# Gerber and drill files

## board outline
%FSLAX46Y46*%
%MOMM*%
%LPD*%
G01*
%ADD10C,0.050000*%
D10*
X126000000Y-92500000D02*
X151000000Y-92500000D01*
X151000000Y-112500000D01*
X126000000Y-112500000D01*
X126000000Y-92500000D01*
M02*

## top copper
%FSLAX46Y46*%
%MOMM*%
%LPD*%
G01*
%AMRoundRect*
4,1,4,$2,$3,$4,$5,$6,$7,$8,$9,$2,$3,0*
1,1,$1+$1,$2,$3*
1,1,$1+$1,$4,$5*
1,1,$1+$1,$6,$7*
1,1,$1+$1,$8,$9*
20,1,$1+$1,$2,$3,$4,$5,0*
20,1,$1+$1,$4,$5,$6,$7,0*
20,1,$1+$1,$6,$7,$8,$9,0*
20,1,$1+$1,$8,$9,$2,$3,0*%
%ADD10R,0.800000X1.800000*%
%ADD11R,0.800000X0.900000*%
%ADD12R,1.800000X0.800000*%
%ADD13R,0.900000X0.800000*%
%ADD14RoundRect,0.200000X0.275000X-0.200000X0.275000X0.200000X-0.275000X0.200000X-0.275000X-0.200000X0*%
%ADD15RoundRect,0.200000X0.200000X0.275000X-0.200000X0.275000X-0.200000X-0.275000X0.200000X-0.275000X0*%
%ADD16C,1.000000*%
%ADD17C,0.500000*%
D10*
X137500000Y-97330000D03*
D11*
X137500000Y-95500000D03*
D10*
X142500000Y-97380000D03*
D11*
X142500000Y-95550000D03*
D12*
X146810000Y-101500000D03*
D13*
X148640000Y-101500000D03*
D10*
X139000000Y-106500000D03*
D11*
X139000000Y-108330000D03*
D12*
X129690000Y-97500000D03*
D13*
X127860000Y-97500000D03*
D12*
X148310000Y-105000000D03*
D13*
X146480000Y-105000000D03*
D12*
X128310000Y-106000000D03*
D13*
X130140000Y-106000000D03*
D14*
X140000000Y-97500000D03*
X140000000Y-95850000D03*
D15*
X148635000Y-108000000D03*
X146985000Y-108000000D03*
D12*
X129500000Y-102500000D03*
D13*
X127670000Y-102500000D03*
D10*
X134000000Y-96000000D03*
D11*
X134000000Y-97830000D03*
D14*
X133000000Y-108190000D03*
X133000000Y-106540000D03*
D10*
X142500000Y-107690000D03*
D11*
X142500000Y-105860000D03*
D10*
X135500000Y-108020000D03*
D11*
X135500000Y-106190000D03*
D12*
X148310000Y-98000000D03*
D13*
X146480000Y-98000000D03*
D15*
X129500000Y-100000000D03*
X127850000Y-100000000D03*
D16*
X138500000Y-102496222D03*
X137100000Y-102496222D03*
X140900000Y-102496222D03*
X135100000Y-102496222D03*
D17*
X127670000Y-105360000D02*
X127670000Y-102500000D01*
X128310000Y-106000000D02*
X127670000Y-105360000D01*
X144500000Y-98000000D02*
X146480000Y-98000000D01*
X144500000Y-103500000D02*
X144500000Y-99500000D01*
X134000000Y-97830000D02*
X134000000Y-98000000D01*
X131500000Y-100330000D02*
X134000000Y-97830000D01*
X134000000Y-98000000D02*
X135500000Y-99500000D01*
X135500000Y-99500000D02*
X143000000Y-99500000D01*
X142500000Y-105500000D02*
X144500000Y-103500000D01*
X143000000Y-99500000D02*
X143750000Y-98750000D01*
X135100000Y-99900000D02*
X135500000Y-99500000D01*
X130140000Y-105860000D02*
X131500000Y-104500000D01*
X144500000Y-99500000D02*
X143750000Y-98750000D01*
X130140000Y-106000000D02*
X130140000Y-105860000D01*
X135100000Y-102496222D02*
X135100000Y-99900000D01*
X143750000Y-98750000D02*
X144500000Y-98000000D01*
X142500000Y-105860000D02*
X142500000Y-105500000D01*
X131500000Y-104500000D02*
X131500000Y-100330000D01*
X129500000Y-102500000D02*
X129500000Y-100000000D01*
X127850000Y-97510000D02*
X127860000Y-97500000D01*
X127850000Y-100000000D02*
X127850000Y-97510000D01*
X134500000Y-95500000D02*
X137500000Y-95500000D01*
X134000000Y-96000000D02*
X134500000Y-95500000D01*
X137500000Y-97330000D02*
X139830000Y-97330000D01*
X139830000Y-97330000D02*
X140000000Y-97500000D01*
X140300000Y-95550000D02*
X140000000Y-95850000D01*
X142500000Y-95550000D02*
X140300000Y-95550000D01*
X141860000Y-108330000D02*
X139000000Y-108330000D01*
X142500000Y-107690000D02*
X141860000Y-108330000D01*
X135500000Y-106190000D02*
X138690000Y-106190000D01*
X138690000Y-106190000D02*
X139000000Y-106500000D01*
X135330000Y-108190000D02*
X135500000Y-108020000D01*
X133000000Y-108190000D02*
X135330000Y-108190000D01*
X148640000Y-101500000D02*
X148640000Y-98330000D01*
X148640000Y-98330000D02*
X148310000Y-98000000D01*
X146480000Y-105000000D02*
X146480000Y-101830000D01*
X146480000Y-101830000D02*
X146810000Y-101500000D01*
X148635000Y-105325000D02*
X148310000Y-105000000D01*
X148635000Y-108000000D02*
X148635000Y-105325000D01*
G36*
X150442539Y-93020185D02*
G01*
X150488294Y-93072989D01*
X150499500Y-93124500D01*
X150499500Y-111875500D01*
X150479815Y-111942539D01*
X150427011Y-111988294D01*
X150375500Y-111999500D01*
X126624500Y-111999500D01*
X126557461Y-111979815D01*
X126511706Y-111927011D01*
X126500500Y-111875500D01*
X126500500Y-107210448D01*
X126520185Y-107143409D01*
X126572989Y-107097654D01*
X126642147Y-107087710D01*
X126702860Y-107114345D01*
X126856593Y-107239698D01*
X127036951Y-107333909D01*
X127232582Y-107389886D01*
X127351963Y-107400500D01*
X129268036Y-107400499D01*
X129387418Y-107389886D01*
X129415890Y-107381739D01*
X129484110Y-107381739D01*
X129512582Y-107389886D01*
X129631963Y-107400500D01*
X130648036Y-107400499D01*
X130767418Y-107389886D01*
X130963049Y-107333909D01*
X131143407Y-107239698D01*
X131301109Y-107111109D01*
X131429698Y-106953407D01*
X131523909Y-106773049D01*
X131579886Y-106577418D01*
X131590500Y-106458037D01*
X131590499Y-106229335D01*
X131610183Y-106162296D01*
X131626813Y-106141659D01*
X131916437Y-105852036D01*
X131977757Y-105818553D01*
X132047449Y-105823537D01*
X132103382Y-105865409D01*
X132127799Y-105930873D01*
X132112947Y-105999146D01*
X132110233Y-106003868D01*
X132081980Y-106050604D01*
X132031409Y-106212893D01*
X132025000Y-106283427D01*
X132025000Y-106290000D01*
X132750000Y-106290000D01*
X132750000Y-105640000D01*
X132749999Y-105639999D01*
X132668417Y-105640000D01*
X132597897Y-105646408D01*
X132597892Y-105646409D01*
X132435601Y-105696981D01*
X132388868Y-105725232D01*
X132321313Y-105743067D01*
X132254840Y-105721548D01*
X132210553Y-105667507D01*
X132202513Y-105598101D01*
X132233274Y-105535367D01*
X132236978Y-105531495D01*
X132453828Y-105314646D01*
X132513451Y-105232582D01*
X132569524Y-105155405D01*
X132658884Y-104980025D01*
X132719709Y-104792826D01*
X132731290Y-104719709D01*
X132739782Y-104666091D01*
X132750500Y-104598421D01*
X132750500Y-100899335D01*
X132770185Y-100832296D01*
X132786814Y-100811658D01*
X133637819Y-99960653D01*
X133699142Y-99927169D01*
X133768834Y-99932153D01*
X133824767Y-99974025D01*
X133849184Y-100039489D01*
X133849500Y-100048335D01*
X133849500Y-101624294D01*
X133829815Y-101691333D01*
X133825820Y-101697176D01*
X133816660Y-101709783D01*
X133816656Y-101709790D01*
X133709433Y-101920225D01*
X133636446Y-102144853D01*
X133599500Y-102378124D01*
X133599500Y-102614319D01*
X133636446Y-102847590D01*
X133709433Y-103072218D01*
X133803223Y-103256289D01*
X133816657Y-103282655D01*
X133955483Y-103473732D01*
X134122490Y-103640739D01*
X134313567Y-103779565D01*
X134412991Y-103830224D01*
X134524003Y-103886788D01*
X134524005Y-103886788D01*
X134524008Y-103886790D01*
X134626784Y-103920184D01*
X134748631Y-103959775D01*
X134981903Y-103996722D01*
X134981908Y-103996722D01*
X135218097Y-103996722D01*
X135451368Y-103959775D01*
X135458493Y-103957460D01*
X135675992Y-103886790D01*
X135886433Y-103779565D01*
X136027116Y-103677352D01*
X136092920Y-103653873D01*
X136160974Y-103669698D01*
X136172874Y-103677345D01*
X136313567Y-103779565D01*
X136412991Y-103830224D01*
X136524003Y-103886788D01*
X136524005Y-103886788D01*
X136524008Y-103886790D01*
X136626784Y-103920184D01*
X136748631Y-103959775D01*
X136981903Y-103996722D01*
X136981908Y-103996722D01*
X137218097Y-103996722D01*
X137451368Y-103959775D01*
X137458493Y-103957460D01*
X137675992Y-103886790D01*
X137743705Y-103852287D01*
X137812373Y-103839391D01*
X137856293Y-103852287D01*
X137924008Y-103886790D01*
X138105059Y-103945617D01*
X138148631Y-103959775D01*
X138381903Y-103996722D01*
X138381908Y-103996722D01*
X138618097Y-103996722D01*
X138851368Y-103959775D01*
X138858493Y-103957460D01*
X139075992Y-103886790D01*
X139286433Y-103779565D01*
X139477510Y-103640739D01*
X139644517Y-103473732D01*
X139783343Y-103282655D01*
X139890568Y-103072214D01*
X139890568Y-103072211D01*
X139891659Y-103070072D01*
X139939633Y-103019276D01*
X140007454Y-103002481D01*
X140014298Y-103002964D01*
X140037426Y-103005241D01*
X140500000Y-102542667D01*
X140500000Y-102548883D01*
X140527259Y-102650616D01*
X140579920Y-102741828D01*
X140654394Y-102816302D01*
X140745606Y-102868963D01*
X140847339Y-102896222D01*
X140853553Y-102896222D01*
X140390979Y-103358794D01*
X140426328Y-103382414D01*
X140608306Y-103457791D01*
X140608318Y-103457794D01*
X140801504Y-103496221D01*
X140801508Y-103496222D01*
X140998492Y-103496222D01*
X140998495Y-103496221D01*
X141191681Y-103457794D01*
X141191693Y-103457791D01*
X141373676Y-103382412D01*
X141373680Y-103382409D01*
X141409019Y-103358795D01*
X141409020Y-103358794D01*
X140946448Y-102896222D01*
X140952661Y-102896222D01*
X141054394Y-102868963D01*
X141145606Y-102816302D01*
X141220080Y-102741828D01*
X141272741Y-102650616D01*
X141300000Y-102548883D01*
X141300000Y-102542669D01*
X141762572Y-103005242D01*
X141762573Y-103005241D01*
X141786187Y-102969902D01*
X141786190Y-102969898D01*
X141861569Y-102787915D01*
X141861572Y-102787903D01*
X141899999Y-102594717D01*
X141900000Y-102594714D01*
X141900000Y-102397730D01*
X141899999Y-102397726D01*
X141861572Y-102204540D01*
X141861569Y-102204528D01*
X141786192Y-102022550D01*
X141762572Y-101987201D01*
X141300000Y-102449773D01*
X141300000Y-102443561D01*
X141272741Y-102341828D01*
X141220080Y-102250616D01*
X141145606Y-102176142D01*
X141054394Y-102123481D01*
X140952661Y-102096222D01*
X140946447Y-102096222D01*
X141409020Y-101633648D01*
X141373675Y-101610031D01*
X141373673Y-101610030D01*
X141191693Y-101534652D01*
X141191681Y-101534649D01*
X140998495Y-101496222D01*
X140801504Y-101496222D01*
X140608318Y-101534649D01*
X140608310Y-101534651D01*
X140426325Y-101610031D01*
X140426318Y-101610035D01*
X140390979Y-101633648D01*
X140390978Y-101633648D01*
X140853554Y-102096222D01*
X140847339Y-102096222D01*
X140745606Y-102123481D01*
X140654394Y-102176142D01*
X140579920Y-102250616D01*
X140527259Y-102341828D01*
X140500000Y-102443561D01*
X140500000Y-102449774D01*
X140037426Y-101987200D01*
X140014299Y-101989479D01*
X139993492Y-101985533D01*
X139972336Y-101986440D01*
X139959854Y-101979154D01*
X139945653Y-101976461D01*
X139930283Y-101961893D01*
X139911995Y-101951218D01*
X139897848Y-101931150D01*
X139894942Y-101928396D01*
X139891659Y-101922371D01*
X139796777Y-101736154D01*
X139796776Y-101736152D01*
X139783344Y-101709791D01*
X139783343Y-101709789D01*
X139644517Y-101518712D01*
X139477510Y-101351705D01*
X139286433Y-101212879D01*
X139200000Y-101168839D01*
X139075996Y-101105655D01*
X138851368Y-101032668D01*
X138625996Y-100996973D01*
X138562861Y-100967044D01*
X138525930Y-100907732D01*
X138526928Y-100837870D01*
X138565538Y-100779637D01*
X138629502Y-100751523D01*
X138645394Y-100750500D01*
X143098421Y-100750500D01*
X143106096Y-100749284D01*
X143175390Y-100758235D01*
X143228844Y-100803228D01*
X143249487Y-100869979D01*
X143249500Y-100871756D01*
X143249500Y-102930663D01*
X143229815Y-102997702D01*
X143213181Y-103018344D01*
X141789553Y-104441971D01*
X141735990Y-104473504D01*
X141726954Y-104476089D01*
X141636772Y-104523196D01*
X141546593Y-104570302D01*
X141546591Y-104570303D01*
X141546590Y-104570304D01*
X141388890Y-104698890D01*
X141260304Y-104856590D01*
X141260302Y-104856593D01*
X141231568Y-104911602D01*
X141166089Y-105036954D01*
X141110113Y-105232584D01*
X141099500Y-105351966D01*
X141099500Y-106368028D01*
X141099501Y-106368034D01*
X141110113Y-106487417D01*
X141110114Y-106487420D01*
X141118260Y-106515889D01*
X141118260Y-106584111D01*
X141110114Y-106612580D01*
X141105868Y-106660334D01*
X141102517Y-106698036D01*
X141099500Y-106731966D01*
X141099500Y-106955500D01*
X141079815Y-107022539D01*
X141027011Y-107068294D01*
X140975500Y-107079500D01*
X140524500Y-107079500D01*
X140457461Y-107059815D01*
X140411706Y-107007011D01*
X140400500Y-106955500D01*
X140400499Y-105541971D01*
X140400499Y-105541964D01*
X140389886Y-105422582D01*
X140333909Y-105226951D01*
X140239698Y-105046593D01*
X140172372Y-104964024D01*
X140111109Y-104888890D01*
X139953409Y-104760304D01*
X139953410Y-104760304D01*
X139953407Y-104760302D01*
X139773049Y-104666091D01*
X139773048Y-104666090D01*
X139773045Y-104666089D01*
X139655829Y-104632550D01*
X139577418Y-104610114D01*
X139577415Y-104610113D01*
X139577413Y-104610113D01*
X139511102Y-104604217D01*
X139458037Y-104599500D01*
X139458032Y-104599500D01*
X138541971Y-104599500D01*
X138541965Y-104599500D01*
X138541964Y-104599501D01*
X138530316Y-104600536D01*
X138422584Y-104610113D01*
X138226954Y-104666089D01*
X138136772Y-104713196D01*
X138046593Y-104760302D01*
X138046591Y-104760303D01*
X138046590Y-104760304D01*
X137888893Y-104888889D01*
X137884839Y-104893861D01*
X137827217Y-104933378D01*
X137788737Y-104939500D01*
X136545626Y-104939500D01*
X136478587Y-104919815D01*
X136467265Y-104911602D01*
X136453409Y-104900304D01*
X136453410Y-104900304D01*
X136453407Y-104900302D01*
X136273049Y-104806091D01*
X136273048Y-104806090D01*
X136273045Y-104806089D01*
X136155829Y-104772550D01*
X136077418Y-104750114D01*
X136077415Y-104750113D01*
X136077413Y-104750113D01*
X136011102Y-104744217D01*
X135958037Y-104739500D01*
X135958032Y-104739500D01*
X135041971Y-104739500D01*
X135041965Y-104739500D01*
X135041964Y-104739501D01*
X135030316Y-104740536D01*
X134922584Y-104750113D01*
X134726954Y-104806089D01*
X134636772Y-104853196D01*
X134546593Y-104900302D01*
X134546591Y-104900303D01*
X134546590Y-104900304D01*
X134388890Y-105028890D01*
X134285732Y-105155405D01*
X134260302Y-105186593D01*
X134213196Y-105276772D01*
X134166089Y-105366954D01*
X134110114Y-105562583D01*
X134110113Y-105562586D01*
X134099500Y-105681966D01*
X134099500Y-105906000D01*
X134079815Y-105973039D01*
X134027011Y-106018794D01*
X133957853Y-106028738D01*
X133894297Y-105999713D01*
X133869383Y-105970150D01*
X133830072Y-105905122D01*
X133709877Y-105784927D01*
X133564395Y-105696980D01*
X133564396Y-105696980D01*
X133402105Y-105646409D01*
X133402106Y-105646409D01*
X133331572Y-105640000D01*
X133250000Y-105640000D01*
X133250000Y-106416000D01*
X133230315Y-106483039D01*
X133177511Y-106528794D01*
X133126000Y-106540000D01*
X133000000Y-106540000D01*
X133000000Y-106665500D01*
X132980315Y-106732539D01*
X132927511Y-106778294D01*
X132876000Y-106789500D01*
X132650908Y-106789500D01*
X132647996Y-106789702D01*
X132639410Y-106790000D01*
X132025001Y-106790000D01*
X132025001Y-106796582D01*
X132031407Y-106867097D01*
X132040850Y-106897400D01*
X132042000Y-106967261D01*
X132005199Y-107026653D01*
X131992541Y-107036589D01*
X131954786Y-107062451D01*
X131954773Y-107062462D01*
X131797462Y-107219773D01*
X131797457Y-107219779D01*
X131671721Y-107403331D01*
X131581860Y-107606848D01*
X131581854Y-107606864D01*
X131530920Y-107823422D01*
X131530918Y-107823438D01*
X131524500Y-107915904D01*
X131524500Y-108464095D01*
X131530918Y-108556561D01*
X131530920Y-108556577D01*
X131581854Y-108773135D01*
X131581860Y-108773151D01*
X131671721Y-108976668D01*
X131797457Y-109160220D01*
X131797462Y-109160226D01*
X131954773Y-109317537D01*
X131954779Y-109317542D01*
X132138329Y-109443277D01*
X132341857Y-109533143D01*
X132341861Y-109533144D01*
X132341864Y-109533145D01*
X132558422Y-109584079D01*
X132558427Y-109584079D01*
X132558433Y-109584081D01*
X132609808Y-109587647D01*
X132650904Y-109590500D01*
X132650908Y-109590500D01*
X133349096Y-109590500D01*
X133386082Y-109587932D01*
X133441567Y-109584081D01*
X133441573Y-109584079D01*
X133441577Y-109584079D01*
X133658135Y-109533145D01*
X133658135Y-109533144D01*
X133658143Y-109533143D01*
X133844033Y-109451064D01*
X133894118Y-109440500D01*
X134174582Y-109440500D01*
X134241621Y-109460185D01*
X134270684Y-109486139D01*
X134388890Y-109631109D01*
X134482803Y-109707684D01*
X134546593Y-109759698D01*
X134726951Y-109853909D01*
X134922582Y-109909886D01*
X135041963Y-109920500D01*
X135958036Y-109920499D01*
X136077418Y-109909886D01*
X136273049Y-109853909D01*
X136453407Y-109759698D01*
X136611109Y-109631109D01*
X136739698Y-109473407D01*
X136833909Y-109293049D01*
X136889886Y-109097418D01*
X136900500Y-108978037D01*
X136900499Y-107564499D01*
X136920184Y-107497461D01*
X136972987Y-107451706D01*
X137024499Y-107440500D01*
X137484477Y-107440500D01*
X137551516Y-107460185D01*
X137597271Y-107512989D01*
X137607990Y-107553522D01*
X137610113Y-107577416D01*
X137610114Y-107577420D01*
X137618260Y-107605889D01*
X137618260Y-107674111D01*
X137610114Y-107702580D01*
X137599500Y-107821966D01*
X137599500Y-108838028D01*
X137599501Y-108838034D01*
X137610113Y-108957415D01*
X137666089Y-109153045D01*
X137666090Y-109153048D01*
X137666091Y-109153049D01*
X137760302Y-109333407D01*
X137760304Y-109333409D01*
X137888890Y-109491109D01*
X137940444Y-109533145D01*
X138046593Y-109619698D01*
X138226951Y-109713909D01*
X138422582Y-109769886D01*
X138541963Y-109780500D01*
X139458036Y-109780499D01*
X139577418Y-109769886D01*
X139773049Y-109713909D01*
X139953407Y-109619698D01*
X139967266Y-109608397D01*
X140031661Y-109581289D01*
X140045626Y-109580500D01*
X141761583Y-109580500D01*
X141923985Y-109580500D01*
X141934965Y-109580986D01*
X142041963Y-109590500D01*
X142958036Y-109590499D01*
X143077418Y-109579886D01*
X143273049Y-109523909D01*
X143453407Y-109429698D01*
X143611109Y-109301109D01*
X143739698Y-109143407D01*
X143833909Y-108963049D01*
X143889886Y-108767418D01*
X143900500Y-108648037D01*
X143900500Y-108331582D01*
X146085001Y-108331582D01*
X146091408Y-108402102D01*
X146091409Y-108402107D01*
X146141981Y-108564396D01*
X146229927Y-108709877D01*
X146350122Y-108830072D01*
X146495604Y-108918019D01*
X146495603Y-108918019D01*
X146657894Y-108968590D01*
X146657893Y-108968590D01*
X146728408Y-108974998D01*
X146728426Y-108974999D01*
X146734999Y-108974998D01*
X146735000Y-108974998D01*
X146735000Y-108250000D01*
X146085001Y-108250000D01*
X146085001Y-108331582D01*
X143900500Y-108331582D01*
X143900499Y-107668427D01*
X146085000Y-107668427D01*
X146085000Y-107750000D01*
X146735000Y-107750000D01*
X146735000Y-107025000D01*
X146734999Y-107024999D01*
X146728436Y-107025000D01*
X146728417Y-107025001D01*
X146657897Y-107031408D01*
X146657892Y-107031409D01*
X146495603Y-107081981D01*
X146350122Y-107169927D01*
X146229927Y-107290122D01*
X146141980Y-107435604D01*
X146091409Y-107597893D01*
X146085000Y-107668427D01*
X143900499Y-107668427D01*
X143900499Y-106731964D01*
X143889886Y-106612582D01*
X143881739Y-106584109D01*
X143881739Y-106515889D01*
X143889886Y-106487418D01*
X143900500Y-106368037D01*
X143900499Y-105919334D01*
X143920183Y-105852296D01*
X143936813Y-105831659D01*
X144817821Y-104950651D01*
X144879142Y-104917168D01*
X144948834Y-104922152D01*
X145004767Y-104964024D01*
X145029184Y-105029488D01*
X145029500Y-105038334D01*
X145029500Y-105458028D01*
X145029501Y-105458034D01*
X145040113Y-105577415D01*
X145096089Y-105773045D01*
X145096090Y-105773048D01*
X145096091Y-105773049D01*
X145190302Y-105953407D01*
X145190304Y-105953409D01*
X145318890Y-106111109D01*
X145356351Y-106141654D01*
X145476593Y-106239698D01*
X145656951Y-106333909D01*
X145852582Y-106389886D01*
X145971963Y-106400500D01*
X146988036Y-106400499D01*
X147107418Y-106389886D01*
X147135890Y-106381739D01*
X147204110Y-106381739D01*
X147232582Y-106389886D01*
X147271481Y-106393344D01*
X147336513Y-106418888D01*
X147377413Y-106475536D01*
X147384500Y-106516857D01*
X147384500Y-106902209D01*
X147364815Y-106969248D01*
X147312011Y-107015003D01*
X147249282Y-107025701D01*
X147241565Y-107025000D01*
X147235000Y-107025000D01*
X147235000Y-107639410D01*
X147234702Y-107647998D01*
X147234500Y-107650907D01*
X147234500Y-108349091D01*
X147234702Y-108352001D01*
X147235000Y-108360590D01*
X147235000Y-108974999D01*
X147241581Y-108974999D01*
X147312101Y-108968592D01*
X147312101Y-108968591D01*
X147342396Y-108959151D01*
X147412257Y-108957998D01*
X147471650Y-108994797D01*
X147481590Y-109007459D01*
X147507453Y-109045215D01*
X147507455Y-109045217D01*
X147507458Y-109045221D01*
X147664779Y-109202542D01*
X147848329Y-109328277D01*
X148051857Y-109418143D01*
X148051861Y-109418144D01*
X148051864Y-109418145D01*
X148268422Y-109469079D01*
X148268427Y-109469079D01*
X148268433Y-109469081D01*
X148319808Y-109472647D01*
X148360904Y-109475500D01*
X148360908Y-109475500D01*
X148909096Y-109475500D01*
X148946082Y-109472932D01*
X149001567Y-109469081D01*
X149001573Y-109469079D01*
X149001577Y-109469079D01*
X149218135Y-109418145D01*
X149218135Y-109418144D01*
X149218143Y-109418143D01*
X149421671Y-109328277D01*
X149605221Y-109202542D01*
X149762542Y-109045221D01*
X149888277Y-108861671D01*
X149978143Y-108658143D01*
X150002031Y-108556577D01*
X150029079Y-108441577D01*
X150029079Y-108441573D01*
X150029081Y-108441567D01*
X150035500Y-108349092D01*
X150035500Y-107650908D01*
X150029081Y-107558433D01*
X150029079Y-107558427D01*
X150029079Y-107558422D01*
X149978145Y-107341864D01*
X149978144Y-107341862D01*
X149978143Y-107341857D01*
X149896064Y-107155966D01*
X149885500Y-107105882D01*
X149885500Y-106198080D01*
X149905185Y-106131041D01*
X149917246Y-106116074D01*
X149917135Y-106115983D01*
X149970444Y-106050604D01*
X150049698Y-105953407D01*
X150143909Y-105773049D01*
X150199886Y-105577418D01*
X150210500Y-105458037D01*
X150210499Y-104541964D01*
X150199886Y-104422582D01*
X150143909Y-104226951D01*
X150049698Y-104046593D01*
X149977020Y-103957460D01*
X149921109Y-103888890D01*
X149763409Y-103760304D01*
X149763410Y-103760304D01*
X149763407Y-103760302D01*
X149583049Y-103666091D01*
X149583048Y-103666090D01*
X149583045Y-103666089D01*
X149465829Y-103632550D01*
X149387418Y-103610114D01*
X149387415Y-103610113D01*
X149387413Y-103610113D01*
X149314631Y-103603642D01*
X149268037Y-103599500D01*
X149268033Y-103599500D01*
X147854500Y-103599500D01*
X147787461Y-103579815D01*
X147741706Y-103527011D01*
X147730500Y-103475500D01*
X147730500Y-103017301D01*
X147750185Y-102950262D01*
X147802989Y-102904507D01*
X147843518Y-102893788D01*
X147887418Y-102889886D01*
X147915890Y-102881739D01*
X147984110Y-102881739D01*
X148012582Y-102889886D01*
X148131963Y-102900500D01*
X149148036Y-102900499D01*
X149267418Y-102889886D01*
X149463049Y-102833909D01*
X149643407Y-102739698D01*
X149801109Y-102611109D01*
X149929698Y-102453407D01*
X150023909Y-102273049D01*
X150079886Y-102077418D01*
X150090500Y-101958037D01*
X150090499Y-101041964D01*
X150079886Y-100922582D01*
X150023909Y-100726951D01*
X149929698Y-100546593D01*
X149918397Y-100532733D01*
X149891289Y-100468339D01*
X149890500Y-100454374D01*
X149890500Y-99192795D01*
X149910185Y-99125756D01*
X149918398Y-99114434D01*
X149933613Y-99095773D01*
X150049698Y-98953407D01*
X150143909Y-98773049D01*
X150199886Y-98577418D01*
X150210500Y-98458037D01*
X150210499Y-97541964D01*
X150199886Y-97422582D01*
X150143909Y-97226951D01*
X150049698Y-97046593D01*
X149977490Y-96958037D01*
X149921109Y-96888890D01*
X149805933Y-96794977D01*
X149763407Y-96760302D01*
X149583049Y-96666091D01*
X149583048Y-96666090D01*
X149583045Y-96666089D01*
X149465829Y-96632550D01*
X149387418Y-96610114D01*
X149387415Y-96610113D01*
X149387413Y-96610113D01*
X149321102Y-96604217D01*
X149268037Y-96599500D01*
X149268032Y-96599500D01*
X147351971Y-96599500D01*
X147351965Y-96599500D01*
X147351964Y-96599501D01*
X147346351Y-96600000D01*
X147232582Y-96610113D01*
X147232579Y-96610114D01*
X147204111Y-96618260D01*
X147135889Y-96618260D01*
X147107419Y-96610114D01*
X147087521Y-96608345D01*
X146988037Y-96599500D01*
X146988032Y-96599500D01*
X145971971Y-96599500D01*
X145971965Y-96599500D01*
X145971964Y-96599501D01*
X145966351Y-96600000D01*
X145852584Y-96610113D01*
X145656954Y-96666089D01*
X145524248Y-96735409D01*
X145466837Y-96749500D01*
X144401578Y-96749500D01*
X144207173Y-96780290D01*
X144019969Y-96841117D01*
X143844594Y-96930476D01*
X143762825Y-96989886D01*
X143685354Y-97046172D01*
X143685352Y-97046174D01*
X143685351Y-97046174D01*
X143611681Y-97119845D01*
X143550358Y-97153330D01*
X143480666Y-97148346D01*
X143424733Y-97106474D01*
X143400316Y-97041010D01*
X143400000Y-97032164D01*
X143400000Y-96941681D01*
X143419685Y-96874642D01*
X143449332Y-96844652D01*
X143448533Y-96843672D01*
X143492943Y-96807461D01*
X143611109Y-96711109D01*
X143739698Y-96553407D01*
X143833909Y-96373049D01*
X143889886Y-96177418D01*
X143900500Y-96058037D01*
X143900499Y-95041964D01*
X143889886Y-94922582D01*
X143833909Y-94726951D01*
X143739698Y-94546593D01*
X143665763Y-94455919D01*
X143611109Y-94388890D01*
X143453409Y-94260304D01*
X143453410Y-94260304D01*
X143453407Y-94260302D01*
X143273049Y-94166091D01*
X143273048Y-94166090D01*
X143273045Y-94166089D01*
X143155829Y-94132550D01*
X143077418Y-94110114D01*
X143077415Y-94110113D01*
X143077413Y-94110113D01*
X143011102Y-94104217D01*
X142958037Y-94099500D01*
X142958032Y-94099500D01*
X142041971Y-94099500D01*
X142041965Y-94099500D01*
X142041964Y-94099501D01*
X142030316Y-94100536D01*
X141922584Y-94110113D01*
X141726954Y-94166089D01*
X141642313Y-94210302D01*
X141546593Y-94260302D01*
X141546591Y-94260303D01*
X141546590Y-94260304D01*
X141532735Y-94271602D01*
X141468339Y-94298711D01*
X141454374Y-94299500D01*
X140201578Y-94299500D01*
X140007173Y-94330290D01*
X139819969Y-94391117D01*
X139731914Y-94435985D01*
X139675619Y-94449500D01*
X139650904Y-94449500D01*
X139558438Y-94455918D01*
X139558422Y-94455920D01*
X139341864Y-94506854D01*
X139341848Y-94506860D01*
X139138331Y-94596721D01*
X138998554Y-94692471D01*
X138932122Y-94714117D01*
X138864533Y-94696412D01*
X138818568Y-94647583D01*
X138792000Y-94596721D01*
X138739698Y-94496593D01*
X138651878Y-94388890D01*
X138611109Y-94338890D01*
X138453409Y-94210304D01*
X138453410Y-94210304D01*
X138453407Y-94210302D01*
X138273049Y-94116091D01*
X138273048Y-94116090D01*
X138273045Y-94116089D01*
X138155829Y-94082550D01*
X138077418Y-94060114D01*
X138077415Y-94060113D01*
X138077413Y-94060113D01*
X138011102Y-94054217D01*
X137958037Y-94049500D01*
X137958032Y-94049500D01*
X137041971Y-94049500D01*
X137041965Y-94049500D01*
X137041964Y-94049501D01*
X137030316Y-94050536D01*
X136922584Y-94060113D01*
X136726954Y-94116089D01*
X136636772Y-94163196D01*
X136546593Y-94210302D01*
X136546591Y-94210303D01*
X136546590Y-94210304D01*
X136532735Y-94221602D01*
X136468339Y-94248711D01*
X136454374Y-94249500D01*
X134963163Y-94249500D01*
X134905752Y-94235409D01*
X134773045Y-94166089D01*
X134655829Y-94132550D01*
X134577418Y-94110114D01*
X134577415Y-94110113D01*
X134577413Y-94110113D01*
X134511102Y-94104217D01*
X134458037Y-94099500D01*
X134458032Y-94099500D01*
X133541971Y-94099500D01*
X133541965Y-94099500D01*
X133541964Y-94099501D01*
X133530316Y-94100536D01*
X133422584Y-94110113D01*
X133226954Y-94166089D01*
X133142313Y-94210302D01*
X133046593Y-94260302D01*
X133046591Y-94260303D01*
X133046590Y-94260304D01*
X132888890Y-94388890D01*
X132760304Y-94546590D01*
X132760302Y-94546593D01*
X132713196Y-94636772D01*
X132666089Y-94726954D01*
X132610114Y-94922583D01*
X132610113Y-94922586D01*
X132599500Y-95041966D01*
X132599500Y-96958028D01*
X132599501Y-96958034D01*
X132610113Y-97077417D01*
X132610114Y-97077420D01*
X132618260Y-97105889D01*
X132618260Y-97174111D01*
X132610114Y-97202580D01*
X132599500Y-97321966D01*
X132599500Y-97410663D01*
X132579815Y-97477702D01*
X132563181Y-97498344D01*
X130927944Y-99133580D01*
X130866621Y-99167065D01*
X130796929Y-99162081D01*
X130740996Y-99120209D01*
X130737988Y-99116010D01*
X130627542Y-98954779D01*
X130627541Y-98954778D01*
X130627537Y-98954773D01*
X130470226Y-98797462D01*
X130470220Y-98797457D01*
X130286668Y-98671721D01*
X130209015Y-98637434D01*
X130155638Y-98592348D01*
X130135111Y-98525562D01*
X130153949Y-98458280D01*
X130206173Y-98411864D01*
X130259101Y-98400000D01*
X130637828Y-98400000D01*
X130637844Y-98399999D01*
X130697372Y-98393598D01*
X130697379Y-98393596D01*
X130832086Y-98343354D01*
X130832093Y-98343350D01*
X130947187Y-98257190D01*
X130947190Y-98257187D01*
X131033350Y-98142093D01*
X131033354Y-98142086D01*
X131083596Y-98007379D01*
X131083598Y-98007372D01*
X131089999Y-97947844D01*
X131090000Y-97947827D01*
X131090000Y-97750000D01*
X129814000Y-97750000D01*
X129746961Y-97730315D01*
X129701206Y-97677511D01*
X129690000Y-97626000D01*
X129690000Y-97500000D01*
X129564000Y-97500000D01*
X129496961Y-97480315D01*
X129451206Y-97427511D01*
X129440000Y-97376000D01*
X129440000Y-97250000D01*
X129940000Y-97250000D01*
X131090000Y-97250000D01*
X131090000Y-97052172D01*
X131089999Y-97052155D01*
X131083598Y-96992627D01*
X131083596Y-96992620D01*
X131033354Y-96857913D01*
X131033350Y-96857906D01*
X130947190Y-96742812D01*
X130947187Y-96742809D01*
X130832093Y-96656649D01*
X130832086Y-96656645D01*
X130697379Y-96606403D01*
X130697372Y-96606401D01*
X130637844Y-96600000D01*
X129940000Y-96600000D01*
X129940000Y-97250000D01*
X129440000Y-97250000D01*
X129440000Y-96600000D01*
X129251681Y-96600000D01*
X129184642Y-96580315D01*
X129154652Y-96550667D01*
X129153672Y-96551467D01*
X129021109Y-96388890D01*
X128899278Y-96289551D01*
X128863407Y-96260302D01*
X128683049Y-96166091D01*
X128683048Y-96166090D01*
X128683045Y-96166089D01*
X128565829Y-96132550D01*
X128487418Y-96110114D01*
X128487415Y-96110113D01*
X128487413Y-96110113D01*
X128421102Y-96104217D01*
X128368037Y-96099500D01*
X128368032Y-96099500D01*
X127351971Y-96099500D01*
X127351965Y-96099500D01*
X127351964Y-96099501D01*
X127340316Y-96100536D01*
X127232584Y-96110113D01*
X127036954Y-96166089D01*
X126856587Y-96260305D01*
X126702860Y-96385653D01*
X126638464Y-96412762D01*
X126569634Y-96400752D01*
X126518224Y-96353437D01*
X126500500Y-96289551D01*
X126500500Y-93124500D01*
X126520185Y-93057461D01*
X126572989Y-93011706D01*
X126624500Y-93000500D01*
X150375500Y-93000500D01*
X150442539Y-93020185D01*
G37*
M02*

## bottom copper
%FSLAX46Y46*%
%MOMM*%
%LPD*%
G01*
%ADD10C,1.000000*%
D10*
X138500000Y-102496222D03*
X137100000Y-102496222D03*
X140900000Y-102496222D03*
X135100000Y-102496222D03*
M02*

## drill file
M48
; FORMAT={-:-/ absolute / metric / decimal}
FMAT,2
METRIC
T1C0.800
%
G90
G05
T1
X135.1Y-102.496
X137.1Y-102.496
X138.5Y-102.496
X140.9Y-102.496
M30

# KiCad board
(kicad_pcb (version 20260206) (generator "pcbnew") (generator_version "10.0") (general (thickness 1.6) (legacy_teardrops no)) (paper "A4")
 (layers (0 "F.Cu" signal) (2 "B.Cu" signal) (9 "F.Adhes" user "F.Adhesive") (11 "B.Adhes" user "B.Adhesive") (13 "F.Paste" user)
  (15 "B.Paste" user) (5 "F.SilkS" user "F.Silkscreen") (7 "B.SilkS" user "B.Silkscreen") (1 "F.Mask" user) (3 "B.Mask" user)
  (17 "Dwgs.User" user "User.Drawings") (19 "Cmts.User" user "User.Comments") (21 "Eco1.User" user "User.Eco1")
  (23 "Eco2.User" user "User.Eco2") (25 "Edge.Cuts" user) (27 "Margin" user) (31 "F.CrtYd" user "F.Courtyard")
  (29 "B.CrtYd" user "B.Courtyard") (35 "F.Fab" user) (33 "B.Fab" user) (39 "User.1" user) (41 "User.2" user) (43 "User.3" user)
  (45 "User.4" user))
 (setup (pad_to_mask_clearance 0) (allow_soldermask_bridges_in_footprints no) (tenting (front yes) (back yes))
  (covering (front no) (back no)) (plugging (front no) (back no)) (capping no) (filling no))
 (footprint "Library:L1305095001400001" (layer "F.Cu") (at 137.5 96.64 -90)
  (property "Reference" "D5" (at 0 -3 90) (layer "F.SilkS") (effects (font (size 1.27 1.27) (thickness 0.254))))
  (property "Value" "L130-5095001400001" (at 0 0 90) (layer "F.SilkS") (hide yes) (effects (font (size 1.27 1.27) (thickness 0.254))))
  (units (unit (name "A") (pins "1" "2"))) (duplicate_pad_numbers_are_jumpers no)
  (pad "1" smd rect (at 0.69 0) (size 0.8 1.8) (layers "F.Cu" "F.Mask" "F.Paste") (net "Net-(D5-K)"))
  (pad "2" smd rect (at -1.14 0) (size 0.8 0.9) (layers "F.Cu" "F.Mask" "F.Paste") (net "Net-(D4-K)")))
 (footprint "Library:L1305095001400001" (layer "F.Cu") (at 142.5 96.69 -90)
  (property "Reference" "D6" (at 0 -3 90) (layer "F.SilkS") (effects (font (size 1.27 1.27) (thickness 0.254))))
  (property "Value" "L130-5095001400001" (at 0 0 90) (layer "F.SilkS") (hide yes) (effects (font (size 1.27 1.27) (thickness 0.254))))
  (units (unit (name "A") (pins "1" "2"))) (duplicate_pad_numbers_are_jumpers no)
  (pad "1" smd rect (at 0.69 0) (size 0.8 1.8) (layers "F.Cu" "F.Mask" "F.Paste") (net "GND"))
  (pad "2" smd rect (at -1.14 0) (size 0.8 0.9) (layers "F.Cu" "F.Mask" "F.Paste") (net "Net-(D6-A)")))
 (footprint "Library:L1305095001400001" (layer "F.Cu") (at 147.5 101.5 180)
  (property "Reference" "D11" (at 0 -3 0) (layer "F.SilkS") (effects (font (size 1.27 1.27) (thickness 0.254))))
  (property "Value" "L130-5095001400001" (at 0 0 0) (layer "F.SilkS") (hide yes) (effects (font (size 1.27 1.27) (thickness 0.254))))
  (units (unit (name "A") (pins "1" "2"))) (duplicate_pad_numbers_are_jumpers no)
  (pad "1" smd rect (at 0.69 0 270) (size 0.8 1.8) (layers "F.Cu" "F.Mask" "F.Paste") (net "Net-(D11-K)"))
  (pad "2" smd rect (at -1.14 0 270) (size 0.8 0.9) (layers "F.Cu" "F.Mask" "F.Paste") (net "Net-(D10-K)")))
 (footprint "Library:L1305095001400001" (layer "F.Cu") (at 139 107.19 90)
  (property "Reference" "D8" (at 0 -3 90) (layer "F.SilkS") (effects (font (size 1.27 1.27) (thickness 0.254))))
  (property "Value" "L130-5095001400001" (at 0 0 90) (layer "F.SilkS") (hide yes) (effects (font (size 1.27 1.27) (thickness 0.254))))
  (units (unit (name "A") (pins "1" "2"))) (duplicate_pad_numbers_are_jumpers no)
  (pad "1" smd rect (at 0.69 0 180) (size 0.8 1.8) (layers "F.Cu" "F.Mask" "F.Paste") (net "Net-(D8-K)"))
  (pad "2" smd rect (at -1.14 0 180) (size 0.8 0.9) (layers "F.Cu" "F.Mask" "F.Paste") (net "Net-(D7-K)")))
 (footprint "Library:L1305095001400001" (layer "F.Cu") (at 129 97.5)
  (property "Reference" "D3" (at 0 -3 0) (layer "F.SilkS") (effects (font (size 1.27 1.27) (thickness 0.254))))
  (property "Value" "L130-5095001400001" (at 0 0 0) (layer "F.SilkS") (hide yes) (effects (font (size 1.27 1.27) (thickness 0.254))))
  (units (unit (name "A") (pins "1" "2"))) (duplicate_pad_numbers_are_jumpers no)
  (pad "1" smd rect (at 0.69 0 90) (size 0.8 1.8) (layers "F.Cu" "F.Mask" "F.Paste") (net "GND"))
  (pad "2" smd rect (at -1.14 0 90) (size 0.8 0.9) (layers "F.Cu" "F.Mask" "F.Paste") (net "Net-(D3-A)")))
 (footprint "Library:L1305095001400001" (layer "F.Cu") (at 147.62 105)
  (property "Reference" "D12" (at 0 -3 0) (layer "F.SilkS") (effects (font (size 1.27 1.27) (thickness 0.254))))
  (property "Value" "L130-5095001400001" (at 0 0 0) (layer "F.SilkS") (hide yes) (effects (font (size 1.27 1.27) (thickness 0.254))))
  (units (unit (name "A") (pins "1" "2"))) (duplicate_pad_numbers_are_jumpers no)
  (pad "1" smd rect (at 0.69 0 90) (size 0.8 1.8) (layers "F.Cu" "F.Mask" "F.Paste") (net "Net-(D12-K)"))
  (pad "2" smd rect (at -1.14 0 90) (size 0.8 0.9) (layers "F.Cu" "F.Mask" "F.Paste") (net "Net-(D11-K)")))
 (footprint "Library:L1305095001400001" (layer "F.Cu") (at 129 106 180)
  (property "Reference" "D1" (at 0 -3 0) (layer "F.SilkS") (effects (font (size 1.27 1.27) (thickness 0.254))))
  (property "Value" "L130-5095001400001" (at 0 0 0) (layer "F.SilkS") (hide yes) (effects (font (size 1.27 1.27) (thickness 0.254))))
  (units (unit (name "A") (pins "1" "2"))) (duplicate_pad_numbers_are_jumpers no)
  (pad "1" smd rect (at 0.69 0 270) (size 0.8 1.8) (layers "F.Cu" "F.Mask" "F.Paste") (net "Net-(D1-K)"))
  (pad "2" smd rect (at -1.14 0 270) (size 0.8 0.9) (layers "F.Cu" "F.Mask" "F.Paste") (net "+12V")))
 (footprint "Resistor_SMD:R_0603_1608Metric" (layer "F.Cu") (at 140 96.675 90)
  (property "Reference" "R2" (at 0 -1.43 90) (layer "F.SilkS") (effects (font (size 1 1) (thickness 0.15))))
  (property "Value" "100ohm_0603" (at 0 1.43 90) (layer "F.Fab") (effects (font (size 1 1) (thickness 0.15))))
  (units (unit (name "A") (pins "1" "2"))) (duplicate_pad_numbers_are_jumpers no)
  (pad "1" smd roundrect (at -0.825 0 90) (size 0.8 0.95) (layers "F.Cu" "F.Mask" "F.Paste") (roundrect_rratio 0.25) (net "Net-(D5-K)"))
  (pad "2" smd roundrect (at 0.825 0 90) (size 0.8 0.95) (layers "F.Cu" "F.Mask" "F.Paste") (roundrect_rratio 0.25) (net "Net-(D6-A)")))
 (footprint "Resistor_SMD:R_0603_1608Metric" (layer "F.Cu") (at 147.81 108 180)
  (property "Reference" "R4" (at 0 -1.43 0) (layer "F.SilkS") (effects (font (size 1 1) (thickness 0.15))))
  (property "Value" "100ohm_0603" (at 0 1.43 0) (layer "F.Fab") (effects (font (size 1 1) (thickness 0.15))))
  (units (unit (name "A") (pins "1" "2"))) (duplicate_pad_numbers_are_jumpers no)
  (pad "1" smd roundrect (at -0.825 0 180) (size 0.8 0.95) (layers "F.Cu" "F.Mask" "F.Paste") (roundrect_rratio 0.25) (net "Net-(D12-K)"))
  (pad "2" smd roundrect (at 0.825 0 180) (size 0.8 0.95) (layers "F.Cu" "F.Mask" "F.Paste") (roundrect_rratio 0.25) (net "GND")))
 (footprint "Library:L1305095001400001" (layer "F.Cu") (at 128.81 102.5)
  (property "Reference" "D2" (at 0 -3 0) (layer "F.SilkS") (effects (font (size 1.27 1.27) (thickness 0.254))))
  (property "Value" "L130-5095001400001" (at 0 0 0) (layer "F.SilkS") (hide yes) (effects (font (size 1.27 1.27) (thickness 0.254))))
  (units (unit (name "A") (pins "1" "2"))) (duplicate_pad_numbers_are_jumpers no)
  (pad "1" smd rect (at 0.69 0 90) (size 0.8 1.8) (layers "F.Cu" "F.Mask" "F.Paste") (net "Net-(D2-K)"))
  (pad "2" smd rect (at -1.14 0 90) (size 0.8 0.9) (layers "F.Cu" "F.Mask" "F.Paste") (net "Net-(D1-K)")))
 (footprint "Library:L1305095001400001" (layer "F.Cu") (at 134 96.69 90)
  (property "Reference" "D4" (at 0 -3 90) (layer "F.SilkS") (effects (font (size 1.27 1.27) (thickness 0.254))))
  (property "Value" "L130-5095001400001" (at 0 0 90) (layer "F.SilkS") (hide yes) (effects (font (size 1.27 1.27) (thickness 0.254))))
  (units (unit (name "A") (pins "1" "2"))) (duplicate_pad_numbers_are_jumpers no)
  (pad "1" smd rect (at 0.69 0 180) (size 0.8 1.8) (layers "F.Cu" "F.Mask" "F.Paste") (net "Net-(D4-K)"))
  (pad "2" smd rect (at -1.14 0 180) (size 0.8 0.9) (layers "F.Cu" "F.Mask" "F.Paste") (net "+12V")))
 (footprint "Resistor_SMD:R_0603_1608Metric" (layer "F.Cu") (at 133 107.365 90)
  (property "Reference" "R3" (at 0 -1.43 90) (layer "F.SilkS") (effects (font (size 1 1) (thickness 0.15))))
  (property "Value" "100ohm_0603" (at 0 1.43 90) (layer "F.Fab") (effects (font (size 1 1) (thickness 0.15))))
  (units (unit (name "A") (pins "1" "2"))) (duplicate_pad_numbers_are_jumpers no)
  (pad "1" smd roundrect (at -0.825 0 90) (size 0.8 0.95) (layers "F.Cu" "F.Mask" "F.Paste") (roundrect_rratio 0.25) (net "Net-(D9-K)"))
  (pad "2" smd roundrect (at 0.825 0 90) (size 0.8 0.95) (layers "F.Cu" "F.Mask" "F.Paste") (roundrect_rratio 0.25) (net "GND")))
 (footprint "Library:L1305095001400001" (layer "F.Cu") (at 142.5 107 -90)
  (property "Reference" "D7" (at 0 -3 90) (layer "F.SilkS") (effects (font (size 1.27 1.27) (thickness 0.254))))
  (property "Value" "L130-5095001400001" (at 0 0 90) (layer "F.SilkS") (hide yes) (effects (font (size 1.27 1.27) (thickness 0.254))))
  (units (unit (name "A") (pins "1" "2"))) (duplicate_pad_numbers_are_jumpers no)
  (pad "1" smd rect (at 0.69 0) (size 0.8 1.8) (layers "F.Cu" "F.Mask" "F.Paste") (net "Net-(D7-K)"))
  (pad "2" smd rect (at -1.14 0) (size 0.8 0.9) (layers "F.Cu" "F.Mask" "F.Paste") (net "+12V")))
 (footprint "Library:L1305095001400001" (layer "F.Cu") (at 135.5 107.33 -90)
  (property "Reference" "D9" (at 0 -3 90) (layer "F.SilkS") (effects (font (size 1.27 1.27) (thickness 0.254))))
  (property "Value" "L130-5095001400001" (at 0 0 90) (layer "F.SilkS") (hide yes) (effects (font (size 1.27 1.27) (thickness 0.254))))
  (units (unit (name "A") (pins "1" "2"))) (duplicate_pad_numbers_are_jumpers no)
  (pad "1" smd rect (at 0.69 0) (size 0.8 1.8) (layers "F.Cu" "F.Mask" "F.Paste") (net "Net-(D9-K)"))
  (pad "2" smd rect (at -1.14 0) (size 0.8 0.9) (layers "F.Cu" "F.Mask" "F.Paste") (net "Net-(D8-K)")))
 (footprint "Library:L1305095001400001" (layer "F.Cu") (at 147.62 98)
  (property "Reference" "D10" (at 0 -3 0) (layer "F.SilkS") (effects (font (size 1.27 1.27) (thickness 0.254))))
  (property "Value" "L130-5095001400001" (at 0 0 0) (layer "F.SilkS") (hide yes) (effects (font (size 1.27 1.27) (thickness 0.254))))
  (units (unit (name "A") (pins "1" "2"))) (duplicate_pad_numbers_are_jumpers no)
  (pad "1" smd rect (at 0.69 0 90) (size 0.8 1.8) (layers "F.Cu" "F.Mask" "F.Paste") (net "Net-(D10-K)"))
  (pad "2" smd rect (at -1.14 0 90) (size 0.8 0.9) (layers "F.Cu" "F.Mask" "F.Paste") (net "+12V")))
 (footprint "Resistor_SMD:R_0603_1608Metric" (layer "F.Cu") (at 128.675 100 180)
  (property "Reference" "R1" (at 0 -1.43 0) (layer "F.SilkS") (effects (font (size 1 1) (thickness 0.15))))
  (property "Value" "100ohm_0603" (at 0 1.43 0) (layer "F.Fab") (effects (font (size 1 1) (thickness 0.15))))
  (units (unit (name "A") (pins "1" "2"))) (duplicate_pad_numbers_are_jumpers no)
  (pad "1" smd roundrect (at -0.825 0 180) (size 0.8 0.95) (layers "F.Cu" "F.Mask" "F.Paste") (roundrect_rratio 0.25) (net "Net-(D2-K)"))
  (pad "2" smd roundrect (at 0.825 0 180) (size 0.8 0.95) (layers "F.Cu" "F.Mask" "F.Paste") (roundrect_rratio 0.25) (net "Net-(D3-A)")))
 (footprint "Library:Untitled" (layer "B.Cu") (at 138.5 102.496222 180)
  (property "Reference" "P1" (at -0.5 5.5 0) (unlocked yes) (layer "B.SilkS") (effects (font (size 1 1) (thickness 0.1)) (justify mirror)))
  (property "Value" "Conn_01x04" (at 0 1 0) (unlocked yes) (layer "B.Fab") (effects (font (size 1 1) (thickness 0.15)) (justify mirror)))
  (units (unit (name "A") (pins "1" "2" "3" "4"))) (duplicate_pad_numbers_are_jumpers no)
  (pad "1" thru_hole circle (at 0 0 180) (size 1 1) (drill 0.8) (layers "*.Cu" "*.Mask") (remove_unused_layers no)
   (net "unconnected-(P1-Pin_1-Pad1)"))
  (pad "2" thru_hole circle (at 1.4 0 180) (size 1 1) (drill 0.8) (layers "*.Cu" "*.Mask") (remove_unused_layers no)
   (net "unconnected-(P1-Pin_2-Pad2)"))
  (pad "3" thru_hole circle (at -2.4 0 180) (size 1 1) (drill 0.8) (layers "*.Cu" "*.Mask") (remove_unused_layers no) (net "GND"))
  (pad "4" thru_hole circle (at 3.4 0 180) (size 1 1) (drill 0.8) (layers "*.Cu" "*.Mask") (remove_unused_layers no) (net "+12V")))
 (gr_rect (start 126 92.5) (end 151 112.5) (stroke (width 0.05) (type default)) (fill no) (layer "Edge.Cuts"))
 (segment (start 127.67 105.36) (end 127.67 102.5) (width 0.5) (layer "F.Cu") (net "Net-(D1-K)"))
 (segment (start 128.31 106) (end 127.67 105.36) (width 0.5) (layer "F.Cu") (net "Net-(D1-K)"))
 (segment (start 144.5 98) (end 146.48 98) (width 0.5) (layer "F.Cu") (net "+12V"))
 (segment (start 144.5 103.5) (end 144.5 99.5) (width 0.5) (layer "F.Cu") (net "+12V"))
 (segment (start 134 97.83) (end 134 98) (width 0.5) (layer "F.Cu") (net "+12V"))
 (segment (start 131.5 100.33) (end 134 97.83) (width 0.5) (layer "F.Cu") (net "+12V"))
 (segment (start 134 98) (end 135.5 99.5) (width 0.5) (layer "F.Cu") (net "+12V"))
 (segment (start 135.5 99.5) (end 143 99.5) (width 0.5) (layer "F.Cu") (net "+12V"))
 (segment (start 142.5 105.5) (end 144.5 103.5) (width 0.5) (layer "F.Cu") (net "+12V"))
 (segment (start 143 99.5) (end 143.75 98.75) (width 0.5) (layer "F.Cu") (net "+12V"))
 (segment (start 135.1 99.9) (end 135.5 99.5) (width 0.5) (layer "F.Cu") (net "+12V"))
 (segment (start 130.14 105.86) (end 131.5 104.5) (width 0.5) (layer "F.Cu") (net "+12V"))
 (segment (start 144.5 99.5) (end 143.75 98.75) (width 0.5) (layer "F.Cu") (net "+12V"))
 (segment (start 130.14 106) (end 130.14 105.86) (width 0.5) (layer "F.Cu") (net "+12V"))
 (segment (start 135.1 102.496222) (end 135.1 99.9) (width 0.5) (layer "F.Cu") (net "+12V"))
 (segment (start 143.75 98.75) (end 144.5 98) (width 0.5) (layer "F.Cu") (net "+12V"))
 (segment (start 142.5 105.86) (end 142.5 105.5) (width 0.5) (layer "F.Cu") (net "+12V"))
 (segment (start 131.5 104.5) (end 131.5 100.33) (width 0.5) (layer "F.Cu") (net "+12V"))
 (segment (start 129.5 102.5) (end 129.5 100) (width 0.5) (layer "F.Cu") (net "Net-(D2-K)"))
 (segment (start 127.85 97.51) (end 127.86 97.5) (width 0.5) (layer "F.Cu") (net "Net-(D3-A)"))
 (segment (start 127.85 100) (end 127.85 97.51) (width 0.5) (layer "F.Cu") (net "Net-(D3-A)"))
 (segment (start 134.5 95.5) (end 137.5 95.5) (width 0.5) (layer "F.Cu") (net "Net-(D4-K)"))
 (segment (start 134 96) (end 134.5 95.5) (width 0.5) (layer "F.Cu") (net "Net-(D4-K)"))
 (segment (start 137.5 97.33) (end 139.83 97.33) (width 0.5) (layer "F.Cu") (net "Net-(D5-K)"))
 (segment (start 139.83 97.33) (end 140 97.5) (width 0.5) (layer "F.Cu") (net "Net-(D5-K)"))
 (segment (start 140.3 95.55) (end 140 95.85) (width 0.5) (layer "F.Cu") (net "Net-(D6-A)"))
 (segment (start 142.5 95.55) (end 140.3 95.55) (width 0.5) (layer "F.Cu") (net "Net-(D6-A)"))
 (segment (start 141.86 108.33) (end 139 108.33) (width 0.5) (layer "F.Cu") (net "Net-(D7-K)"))
 (segment (start 142.5 107.69) (end 141.86 108.33) (width 0.5) (layer "F.Cu") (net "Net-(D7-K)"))
 (segment (start 135.5 106.19) (end 138.69 106.19) (width 0.5) (layer "F.Cu") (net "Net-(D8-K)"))
 (segment (start 138.69 106.19) (end 139 106.5) (width 0.5) (layer "F.Cu") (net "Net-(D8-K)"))
 (segment (start 135.33 108.19) (end 135.5 108.02) (width 0.5) (layer "F.Cu") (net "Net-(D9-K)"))
 (segment (start 133 108.19) (end 135.33 108.19) (width 0.5) (layer "F.Cu") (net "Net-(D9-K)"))
 (segment (start 148.64 101.5) (end 148.64 98.33) (width 0.5) (layer "F.Cu") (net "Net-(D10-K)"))
 (segment (start 148.64 98.33) (end 148.31 98) (width 0.5) (layer "F.Cu") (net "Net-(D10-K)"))
 (segment (start 146.48 105) (end 146.48 101.83) (width 0.5) (layer "F.Cu") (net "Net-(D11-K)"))
 (segment (start 146.48 101.83) (end 146.81 101.5) (width 0.5) (layer "F.Cu") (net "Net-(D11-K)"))
 (segment (start 148.635 105.325) (end 148.31 105) (width 0.5) (layer "F.Cu") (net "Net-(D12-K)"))
 (segment (start 148.635 108) (end 148.635 105.325) (width 0.5) (layer "F.Cu") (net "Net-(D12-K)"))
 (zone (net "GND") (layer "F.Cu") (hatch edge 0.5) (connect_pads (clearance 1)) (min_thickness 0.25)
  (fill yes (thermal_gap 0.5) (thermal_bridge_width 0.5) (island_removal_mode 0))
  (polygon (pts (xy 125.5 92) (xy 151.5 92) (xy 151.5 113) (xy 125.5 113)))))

